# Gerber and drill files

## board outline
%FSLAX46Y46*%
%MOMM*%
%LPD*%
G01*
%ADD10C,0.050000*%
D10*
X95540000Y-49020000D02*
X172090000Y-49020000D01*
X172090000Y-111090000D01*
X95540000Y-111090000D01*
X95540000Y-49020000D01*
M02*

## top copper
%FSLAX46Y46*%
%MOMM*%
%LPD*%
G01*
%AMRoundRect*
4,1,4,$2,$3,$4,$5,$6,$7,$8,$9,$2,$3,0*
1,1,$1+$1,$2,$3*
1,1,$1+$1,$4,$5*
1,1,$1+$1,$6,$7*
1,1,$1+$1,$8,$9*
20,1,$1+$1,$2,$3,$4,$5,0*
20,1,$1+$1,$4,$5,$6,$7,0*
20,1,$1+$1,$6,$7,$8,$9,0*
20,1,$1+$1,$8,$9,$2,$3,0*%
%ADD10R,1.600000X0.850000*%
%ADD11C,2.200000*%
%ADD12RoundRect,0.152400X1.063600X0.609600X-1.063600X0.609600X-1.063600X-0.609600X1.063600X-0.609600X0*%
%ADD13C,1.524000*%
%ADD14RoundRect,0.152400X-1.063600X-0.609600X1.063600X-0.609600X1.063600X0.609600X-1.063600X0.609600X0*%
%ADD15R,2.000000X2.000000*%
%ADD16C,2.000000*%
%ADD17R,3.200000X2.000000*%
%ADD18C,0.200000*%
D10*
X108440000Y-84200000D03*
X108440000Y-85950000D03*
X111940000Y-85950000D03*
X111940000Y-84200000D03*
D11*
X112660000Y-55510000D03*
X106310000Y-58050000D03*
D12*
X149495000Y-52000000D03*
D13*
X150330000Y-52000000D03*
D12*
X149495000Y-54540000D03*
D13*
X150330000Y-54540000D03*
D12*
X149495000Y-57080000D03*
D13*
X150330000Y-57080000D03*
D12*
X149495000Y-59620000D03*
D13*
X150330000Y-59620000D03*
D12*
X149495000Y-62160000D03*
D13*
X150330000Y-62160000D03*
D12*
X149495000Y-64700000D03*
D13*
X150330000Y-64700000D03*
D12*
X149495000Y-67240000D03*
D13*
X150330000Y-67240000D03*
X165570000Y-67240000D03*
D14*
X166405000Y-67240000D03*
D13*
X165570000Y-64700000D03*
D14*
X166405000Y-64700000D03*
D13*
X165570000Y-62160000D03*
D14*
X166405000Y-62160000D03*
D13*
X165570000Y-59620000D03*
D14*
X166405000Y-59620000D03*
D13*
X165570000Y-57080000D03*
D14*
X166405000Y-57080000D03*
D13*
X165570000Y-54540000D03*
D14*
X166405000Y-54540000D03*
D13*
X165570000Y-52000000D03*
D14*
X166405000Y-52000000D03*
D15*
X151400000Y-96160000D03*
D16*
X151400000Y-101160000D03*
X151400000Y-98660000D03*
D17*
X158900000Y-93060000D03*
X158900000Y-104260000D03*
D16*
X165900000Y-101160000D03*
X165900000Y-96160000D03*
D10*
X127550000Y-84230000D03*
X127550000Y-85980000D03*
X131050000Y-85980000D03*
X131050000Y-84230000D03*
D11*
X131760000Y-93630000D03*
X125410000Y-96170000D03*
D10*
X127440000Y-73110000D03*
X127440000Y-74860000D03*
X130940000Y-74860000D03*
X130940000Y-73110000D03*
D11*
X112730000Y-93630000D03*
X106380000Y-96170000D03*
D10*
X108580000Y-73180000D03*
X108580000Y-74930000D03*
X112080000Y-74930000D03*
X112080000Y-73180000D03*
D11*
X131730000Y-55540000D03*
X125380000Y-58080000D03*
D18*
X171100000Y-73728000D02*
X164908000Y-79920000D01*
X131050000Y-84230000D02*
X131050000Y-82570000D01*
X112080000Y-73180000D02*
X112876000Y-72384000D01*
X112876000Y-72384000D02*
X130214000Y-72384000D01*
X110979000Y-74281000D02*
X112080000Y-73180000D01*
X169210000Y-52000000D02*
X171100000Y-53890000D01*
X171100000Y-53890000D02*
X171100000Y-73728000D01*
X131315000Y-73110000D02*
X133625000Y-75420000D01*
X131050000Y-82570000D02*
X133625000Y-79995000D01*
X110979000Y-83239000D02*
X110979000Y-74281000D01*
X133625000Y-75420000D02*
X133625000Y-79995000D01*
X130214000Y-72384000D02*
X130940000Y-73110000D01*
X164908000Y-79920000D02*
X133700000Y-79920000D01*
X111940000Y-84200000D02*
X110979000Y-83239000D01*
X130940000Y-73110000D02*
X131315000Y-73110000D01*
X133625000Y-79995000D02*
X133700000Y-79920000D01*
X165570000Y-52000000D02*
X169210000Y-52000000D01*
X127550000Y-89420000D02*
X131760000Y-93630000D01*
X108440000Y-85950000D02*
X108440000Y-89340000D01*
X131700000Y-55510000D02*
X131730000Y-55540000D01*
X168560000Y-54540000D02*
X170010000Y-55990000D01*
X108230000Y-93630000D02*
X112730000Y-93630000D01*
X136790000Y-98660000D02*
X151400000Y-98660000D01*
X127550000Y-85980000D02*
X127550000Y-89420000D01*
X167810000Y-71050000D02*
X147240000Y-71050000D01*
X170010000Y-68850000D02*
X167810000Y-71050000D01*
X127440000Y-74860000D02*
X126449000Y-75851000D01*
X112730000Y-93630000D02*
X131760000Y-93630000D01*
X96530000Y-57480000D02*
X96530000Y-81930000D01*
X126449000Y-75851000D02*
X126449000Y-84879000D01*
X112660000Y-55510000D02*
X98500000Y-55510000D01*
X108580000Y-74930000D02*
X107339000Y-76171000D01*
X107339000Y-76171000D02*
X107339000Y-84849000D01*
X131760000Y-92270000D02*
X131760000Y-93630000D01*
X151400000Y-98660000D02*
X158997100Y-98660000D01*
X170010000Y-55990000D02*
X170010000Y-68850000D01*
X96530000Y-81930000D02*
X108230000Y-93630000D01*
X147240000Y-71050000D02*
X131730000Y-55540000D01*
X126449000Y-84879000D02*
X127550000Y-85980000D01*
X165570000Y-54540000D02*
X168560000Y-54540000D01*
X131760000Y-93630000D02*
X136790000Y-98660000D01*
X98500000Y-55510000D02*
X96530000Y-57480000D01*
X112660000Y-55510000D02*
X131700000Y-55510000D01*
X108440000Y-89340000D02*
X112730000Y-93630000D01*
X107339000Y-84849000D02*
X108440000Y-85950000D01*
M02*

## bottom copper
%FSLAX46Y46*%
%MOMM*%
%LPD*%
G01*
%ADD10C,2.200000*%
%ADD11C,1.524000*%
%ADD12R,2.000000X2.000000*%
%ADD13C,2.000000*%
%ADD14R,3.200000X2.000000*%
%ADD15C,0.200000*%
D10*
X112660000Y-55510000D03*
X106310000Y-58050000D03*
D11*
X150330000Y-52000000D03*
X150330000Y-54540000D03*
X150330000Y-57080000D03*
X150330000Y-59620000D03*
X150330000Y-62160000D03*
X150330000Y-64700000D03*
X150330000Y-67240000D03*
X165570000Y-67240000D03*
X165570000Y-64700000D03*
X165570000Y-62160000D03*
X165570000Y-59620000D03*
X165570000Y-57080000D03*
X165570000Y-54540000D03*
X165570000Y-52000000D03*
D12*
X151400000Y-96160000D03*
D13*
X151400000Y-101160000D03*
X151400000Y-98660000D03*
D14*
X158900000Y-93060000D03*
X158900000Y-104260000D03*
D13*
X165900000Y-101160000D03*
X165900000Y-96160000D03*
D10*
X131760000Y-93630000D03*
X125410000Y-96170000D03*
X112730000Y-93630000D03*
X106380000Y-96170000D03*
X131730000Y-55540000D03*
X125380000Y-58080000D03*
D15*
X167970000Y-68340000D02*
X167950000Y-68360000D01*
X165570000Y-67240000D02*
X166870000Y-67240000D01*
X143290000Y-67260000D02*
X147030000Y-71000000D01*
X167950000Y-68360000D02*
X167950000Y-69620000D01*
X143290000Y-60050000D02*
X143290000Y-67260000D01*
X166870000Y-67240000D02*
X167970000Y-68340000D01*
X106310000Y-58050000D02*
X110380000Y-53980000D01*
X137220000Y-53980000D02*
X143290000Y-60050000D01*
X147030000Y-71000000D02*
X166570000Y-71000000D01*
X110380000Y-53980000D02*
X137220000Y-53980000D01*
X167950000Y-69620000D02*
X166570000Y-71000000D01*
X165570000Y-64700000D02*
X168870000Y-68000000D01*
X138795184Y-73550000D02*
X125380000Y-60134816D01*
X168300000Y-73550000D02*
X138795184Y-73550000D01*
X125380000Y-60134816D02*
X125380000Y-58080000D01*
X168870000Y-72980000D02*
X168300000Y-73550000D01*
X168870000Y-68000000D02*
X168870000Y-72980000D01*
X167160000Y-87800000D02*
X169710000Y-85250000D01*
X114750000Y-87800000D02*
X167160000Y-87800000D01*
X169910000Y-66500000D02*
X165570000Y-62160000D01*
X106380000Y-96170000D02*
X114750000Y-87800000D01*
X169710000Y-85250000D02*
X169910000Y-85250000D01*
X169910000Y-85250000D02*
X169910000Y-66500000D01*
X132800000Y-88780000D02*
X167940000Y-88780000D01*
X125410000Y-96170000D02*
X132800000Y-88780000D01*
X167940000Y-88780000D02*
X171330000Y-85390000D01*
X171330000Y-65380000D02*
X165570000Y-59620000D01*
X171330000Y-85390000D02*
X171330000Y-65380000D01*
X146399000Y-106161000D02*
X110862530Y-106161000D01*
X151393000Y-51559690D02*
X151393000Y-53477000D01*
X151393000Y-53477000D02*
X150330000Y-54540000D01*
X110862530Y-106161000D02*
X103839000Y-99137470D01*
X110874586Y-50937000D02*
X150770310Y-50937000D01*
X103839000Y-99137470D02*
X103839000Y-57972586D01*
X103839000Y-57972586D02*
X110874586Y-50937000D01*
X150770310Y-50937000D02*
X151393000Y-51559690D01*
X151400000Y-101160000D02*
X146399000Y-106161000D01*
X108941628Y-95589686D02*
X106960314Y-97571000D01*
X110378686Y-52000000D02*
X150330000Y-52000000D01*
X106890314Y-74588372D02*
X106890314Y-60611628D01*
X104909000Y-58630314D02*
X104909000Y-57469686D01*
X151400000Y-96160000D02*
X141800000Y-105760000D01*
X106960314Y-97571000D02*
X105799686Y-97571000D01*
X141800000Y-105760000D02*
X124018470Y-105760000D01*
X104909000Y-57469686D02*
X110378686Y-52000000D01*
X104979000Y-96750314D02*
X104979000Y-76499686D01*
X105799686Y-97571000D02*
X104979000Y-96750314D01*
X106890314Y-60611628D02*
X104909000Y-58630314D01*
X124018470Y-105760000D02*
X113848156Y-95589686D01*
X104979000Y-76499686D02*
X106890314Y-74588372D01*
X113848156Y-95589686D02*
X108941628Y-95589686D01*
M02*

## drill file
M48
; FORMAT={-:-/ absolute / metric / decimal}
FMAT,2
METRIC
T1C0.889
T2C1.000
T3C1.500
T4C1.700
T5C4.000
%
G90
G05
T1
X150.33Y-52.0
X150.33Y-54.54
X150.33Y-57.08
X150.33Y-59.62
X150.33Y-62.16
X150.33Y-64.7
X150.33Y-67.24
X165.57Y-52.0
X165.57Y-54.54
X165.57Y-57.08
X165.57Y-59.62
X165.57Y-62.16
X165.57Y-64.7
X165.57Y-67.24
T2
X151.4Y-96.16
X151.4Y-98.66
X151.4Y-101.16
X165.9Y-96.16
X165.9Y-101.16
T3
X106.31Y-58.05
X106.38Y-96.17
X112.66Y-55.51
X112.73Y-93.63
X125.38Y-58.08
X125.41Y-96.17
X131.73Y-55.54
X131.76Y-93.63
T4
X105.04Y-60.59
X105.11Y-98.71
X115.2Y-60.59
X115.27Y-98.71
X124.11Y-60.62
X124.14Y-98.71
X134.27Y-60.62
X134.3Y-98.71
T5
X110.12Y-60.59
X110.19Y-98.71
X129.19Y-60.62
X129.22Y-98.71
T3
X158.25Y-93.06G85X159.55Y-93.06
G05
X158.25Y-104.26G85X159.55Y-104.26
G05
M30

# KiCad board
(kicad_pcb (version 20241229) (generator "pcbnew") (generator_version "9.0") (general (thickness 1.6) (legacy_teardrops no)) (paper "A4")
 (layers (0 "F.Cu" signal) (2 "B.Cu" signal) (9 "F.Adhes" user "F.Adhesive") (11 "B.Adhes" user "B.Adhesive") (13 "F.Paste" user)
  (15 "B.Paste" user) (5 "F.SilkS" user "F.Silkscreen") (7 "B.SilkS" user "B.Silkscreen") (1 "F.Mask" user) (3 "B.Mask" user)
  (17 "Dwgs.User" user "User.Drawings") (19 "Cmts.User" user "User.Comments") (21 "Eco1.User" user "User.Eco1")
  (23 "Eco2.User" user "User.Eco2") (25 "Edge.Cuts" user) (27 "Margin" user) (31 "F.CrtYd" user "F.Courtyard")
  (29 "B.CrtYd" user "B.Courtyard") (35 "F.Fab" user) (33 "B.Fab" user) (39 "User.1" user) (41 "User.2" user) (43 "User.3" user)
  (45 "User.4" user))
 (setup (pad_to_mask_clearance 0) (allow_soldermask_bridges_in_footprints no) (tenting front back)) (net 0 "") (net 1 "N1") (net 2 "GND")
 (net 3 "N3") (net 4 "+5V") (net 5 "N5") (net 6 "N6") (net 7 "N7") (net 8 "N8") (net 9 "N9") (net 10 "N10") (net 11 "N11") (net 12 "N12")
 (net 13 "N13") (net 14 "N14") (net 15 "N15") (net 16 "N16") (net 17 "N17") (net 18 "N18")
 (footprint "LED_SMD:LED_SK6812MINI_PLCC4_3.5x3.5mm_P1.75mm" (layer "F.Cu") (at 110.19 85.075)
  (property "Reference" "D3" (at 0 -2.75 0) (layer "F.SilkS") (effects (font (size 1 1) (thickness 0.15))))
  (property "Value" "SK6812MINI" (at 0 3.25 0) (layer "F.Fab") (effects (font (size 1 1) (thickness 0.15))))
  (pad "1" smd rect (at -1.75 -0.875) (size 1.6 0.85) (layers "F.Cu" "F.Mask" "F.Paste") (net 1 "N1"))
  (pad "2" smd rect (at -1.75 0.875) (size 1.6 0.85) (layers "F.Cu" "F.Mask" "F.Paste") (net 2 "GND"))
  (pad "3" smd rect (at 1.75 0.875) (size 1.6 0.85) (layers "F.Cu" "F.Mask" "F.Paste") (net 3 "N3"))
  (pad "4" smd rect (at 1.75 -0.875) (size 1.6 0.85) (layers "F.Cu" "F.Mask" "F.Paste") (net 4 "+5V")))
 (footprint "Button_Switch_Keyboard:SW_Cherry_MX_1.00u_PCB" (layer "F.Cu") (at 112.66 55.51)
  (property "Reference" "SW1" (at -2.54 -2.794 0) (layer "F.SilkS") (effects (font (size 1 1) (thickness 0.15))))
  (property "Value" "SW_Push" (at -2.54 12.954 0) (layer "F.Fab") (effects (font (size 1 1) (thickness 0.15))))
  (pad "" np_thru_hole circle (at -7.62 5.08) (size 1.7 1.7) (drill 1.7) (layers "*.Cu" "*.Mask"))
  (pad "" np_thru_hole circle (at -2.54 5.08) (size 4 4) (drill 4) (layers "*.Cu" "*.Mask"))
  (pad "" np_thru_hole circle (at 2.54 5.08) (size 1.7 1.7) (drill 1.7) (layers "*.Cu" "*.Mask"))
  (pad "1" thru_hole circle (at 0 0) (size 2.2 2.2) (drill 1.5) (layers "*.Cu" "*.Mask") (remove_unused_layers no) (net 2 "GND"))
  (pad "2" thru_hole circle (at -6.35 2.54) (size 2.2 2.2) (drill 1.5) (layers "*.Cu" "*.Mask") (remove_unused_layers no) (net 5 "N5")))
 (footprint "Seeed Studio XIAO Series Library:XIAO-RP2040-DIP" (layer "F.Cu") (at 157.95 59.62)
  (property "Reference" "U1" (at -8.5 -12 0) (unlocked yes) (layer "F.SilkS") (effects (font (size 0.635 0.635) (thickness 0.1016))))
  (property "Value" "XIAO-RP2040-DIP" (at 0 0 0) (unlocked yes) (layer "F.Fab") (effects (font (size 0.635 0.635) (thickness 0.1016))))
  (pad "1" smd roundrect (at -8.455 -7.62 180) (size 2.432 1.524) (layers "F.Cu" "F.Mask") (roundrect_rratio 0.1) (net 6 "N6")
   (thermal_bridge_angle 45))
  (pad "1" thru_hole circle (at -7.62 -7.62 180) (size 1.524 1.524) (drill 0.889) (layers "*.Cu" "*.Mask") (remove_unused_layers no)
   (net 6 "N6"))
  (pad "2" smd roundrect (at -8.455 -5.08 180) (size 2.432 1.524) (layers "F.Cu" "F.Mask") (roundrect_rratio 0.1) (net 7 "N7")
   (thermal_bridge_angle 45))
  (pad "2" thru_hole circle (at -7.62 -5.08 180) (size 1.524 1.524) (drill 0.889) (layers "*.Cu" "*.Mask") (remove_unused_layers no)
   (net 7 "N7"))
  (pad "3" smd roundrect (at -8.455 -2.54 180) (size 2.432 1.524) (layers "F.Cu" "F.Mask") (roundrect_rratio 0.1) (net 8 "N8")
   (thermal_bridge_angle 45))
  (pad "3" thru_hole circle (at -7.62 -2.54 180) (size 1.524 1.524) (drill 0.889) (layers "*.Cu" "*.Mask") (remove_unused_layers no)
   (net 8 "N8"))
  (pad "4" smd roundrect (at -8.455 0 180) (size 2.432 1.524) (layers "F.Cu" "F.Mask") (roundrect_rratio 0.1) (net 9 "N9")
   (thermal_bridge_angle 45))
  (pad "4" thru_hole circle (at -7.62 0 180) (size 1.524 1.524) (drill 0.889) (layers "*.Cu" "*.Mask") (remove_unused_layers no)
   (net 9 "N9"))
  (pad "5" smd roundrect (at -8.455 2.54 180) (size 2.432 1.524) (layers "F.Cu" "F.Mask") (roundrect_rratio 0.1) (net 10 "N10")
   (thermal_bridge_angle 45))
  (pad "5" thru_hole circle (at -7.62 2.54 180) (size 1.524 1.524) (drill 0.889) (layers "*.Cu" "*.Mask") (remove_unused_layers no)
   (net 10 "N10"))
  (pad "6" smd roundrect (at -8.455 5.08 180) (size 2.432 1.524) (layers "F.Cu" "F.Mask") (roundrect_rratio 0.1) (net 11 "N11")
   (thermal_bridge_angle 45))
  (pad "6" thru_hole circle (at -7.62 5.08 180) (size 1.524 1.524) (drill 0.889) (layers "*.Cu" "*.Mask") (remove_unused_layers no)
   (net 11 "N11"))
  (pad "7" smd roundrect (at -8.455 7.62 180) (size 2.432 1.524) (layers "F.Cu" "F.Mask") (roundrect_rratio 0.1) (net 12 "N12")
   (thermal_bridge_angle 45))
  (pad "7" thru_hole circle (at -7.62 7.62 180) (size 1.524 1.524) (drill 0.889) (layers "*.Cu" "*.Mask") (remove_unused_layers no)
   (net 12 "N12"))
  (pad "8" thru_hole circle (at 7.62 7.62) (size 1.524 1.524) (drill 0.889) (layers "*.Cu" "*.Mask") (remove_unused_layers no) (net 5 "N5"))
  (pad "8" smd roundrect (at 8.455 7.62) (size 2.432 1.524) (layers "F.Cu" "F.Mask") (roundrect_rratio 0.1) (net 5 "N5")
   (thermal_bridge_angle 45))
  (pad "9" thru_hole circle (at 7.62 5.08) (size 1.524 1.524) (drill 0.889) (layers "*.Cu" "*.Mask") (remove_unused_layers no)
   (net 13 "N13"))
  (pad "9" smd roundrect (at 8.455 5.08) (size 2.432 1.524) (layers "F.Cu" "F.Mask") (roundrect_rratio 0.1) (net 13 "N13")
   (thermal_bridge_angle 45))
  (pad "10" thru_hole circle (at 7.62 2.54) (size 1.524 1.524) (drill 0.889) (layers "*.Cu" "*.Mask") (remove_unused_layers no)
   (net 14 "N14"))
  (pad "10" smd roundrect (at 8.455 2.54) (size 2.432 1.524) (layers "F.Cu" "F.Mask") (roundrect_rratio 0.1) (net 14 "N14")
   (thermal_bridge_angle 45))
  (pad "11" thru_hole circle (at 7.62 0) (size 1.524 1.524) (drill 0.889) (layers "*.Cu" "*.Mask") (remove_unused_layers no) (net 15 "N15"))
  (pad "11" smd roundrect (at 8.455 0) (size 2.432 1.524) (layers "F.Cu" "F.Mask") (roundrect_rratio 0.1) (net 15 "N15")
   (thermal_bridge_angle 45))
  (pad "12" thru_hole circle (at 7.62 -2.54) (size 1.524 1.524) (drill 0.889) (layers "*.Cu" "*.Mask") (remove_unused_layers no)
   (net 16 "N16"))
  (pad "12" smd roundrect (at 8.455 -2.54) (size 2.432 1.524) (layers "F.Cu" "F.Mask") (roundrect_rratio 0.1) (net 16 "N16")
   (thermal_bridge_angle 45))
  (pad "13" thru_hole circle (at 7.62 -5.08) (size 1.524 1.524) (drill 0.889) (layers "*.Cu" "*.Mask") (remove_unused_layers no)
   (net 2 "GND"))
  (pad "13" smd roundrect (at 8.455 -5.08) (size 2.432 1.524) (layers "F.Cu" "F.Mask") (roundrect_rratio 0.1) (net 2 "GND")
   (thermal_bridge_angle 45))
  (pad "14" thru_hole circle (at 7.62 -7.62) (size 1.524 1.524) (drill 0.889) (layers "*.Cu" "*.Mask") (remove_unused_layers no)
   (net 4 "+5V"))
  (pad "14" smd roundrect (at 8.455 -7.62) (size 2.432 1.524) (layers "F.Cu" "F.Mask") (roundrect_rratio 0.1) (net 4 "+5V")
   (thermal_bridge_angle 45)))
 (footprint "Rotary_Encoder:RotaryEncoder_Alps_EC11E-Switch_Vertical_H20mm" (layer "F.Cu") (at 151.4 96.16)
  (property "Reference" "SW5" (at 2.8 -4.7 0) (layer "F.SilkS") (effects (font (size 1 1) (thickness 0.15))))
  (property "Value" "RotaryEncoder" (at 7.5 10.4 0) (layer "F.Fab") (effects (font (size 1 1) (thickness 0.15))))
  (pad "A" thru_hole rect (at 0 0) (size 2 2) (drill 1) (layers "*.Cu" "*.Mask") (remove_unused_layers no) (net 6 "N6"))
  (pad "B" thru_hole circle (at 0 5) (size 2 2) (drill 1) (layers "*.Cu" "*.Mask") (remove_unused_layers no) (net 7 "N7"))
  (pad "C" thru_hole circle (at 0 2.5) (size 2 2) (drill 1) (layers "*.Cu" "*.Mask") (remove_unused_layers no) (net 2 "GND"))
  (pad "MP" thru_hole rect (at 7.5 -3.1) (size 3.2 2) (drill oval 2.8 1.5) (layers "*.Cu" "*.Mask") (remove_unused_layers no))
  (pad "MP" thru_hole rect (at 7.5 8.1) (size 3.2 2) (drill oval 2.8 1.5) (layers "*.Cu" "*.Mask") (remove_unused_layers no))
  (pad "S1" thru_hole circle (at 14.5 5) (size 2 2) (drill 1) (layers "*.Cu" "*.Mask") (remove_unused_layers no))
  (pad "S2" thru_hole circle (at 14.5 0) (size 2 2) (drill 1) (layers "*.Cu" "*.Mask") (remove_unused_layers no)))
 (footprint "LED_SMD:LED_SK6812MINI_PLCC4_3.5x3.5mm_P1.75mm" (layer "F.Cu") (at 129.3 85.105)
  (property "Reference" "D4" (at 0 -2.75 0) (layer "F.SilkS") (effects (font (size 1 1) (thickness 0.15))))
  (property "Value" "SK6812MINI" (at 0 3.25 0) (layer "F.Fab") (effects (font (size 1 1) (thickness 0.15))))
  (pad "1" smd rect (at -1.75 -0.875) (size 1.6 0.85) (layers "F.Cu" "F.Mask" "F.Paste") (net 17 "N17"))
  (pad "2" smd rect (at -1.75 0.875) (size 1.6 0.85) (layers "F.Cu" "F.Mask" "F.Paste") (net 2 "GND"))
  (pad "3" smd rect (at 1.75 0.875) (size 1.6 0.85) (layers "F.Cu" "F.Mask" "F.Paste") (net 1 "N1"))
  (pad "4" smd rect (at 1.75 -0.875) (size 1.6 0.85) (layers "F.Cu" "F.Mask" "F.Paste") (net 4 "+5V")))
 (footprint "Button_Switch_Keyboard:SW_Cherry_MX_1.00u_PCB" (layer "F.Cu") (at 131.76 93.63)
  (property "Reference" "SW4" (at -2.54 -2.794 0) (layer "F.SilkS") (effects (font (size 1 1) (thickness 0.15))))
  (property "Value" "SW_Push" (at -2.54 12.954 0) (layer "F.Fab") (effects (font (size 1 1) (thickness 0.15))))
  (pad "" np_thru_hole circle (at -7.62 5.08) (size 1.7 1.7) (drill 1.7) (layers "*.Cu" "*.Mask"))
  (pad "" np_thru_hole circle (at -2.54 5.08) (size 4 4) (drill 4) (layers "*.Cu" "*.Mask"))
  (pad "" np_thru_hole circle (at 2.54 5.08) (size 1.7 1.7) (drill 1.7) (layers "*.Cu" "*.Mask"))
  (pad "1" thru_hole circle (at 0 0) (size 2.2 2.2) (drill 1.5) (layers "*.Cu" "*.Mask") (remove_unused_layers no) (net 2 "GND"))
  (pad "2" thru_hole circle (at -6.35 2.54) (size 2.2 2.2) (drill 1.5) (layers "*.Cu" "*.Mask") (remove_unused_layers no) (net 15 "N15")))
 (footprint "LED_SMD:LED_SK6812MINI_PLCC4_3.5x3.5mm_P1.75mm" (layer "F.Cu") (at 129.19 73.985)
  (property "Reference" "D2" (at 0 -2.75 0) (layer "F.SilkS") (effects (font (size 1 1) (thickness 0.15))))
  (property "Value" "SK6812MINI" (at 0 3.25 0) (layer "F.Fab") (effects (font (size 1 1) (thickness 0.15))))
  (pad "1" smd rect (at -1.75 -0.875) (size 1.6 0.85) (layers "F.Cu" "F.Mask" "F.Paste") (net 3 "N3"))
  (pad "2" smd rect (at -1.75 0.875) (size 1.6 0.85) (layers "F.Cu" "F.Mask" "F.Paste") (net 2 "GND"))
  (pad "3" smd rect (at 1.75 0.875) (size 1.6 0.85) (layers "F.Cu" "F.Mask" "F.Paste") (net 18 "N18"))
  (pad "4" smd rect (at 1.75 -0.875) (size 1.6 0.85) (layers "F.Cu" "F.Mask" "F.Paste") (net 4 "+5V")))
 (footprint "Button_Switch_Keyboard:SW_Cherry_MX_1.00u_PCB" (layer "F.Cu") (at 112.73 93.63)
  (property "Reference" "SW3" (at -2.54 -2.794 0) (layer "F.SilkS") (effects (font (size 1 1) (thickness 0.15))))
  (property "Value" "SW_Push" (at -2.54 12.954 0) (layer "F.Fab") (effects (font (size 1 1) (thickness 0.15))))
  (pad "" np_thru_hole circle (at -7.62 5.08) (size 1.7 1.7) (drill 1.7) (layers "*.Cu" "*.Mask"))
  (pad "" np_thru_hole circle (at -2.54 5.08) (size 4 4) (drill 4) (layers "*.Cu" "*.Mask"))
  (pad "" np_thru_hole circle (at 2.54 5.08) (size 1.7 1.7) (drill 1.7) (layers "*.Cu" "*.Mask"))
  (pad "1" thru_hole circle (at 0 0) (size 2.2 2.2) (drill 1.5) (layers "*.Cu" "*.Mask") (remove_unused_layers no) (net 2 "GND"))
  (pad "2" thru_hole circle (at -6.35 2.54) (size 2.2 2.2) (drill 1.5) (layers "*.Cu" "*.Mask") (remove_unused_layers no) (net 14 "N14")))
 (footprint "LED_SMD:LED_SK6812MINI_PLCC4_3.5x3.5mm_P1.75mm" (layer "F.Cu") (at 110.33 74.055)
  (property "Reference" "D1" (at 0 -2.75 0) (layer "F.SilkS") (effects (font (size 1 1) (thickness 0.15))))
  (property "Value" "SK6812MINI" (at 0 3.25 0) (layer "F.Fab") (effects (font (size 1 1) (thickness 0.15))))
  (pad "1" smd rect (at -1.75 -0.875) (size 1.6 0.85) (layers "F.Cu" "F.Mask" "F.Paste") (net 18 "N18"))
  (pad "2" smd rect (at -1.75 0.875) (size 1.6 0.85) (layers "F.Cu" "F.Mask" "F.Paste") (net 2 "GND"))
  (pad "3" smd rect (at 1.75 0.875) (size 1.6 0.85) (layers "F.Cu" "F.Mask" "F.Paste") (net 10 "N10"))
  (pad "4" smd rect (at 1.75 -0.875) (size 1.6 0.85) (layers "F.Cu" "F.Mask" "F.Paste") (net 4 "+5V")))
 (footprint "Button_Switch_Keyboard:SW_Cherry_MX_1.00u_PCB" (layer "F.Cu") (at 131.73 55.54)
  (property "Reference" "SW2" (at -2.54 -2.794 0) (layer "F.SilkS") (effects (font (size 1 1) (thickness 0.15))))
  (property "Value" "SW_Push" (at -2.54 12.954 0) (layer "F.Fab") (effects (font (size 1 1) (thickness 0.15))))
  (pad "" np_thru_hole circle (at -7.62 5.08) (size 1.7 1.7) (drill 1.7) (layers "*.Cu" "*.Mask"))
  (pad "" np_thru_hole circle (at -2.54 5.08) (size 4 4) (drill 4) (layers "*.Cu" "*.Mask"))
  (pad "" np_thru_hole circle (at 2.54 5.08) (size 1.7 1.7) (drill 1.7) (layers "*.Cu" "*.Mask"))
  (pad "1" thru_hole circle (at 0 0) (size 2.2 2.2) (drill 1.5) (layers "*.Cu" "*.Mask") (remove_unused_layers no) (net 2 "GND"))
  (pad "2" thru_hole circle (at -6.35 2.54) (size 2.2 2.2) (drill 1.5) (layers "*.Cu" "*.Mask") (remove_unused_layers no) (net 13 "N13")))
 (gr_rect (start 95.54 49.02) (end 172.09 111.09) (stroke (width 0.05) (type default)) (fill no) (layer "Edge.Cuts"))
 (segment (start 171.1 73.728) (end 164.908 79.92) (width 0.2) (layer "F.Cu") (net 4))
 (segment (start 131.05 84.23) (end 131.05 82.57) (width 0.2) (layer "F.Cu") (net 4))
 (segment (start 112.08 73.18) (end 112.876 72.384) (width 0.2) (layer "F.Cu") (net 4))
 (segment (start 112.876 72.384) (end 130.214 72.384) (width 0.2) (layer "F.Cu") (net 4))
 (segment (start 110.979 74.281) (end 112.08 73.18) (width 0.2) (layer "F.Cu") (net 4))
 (segment (start 169.21 52) (end 171.1 53.89) (width 0.2) (layer "F.Cu") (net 4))
 (segment (start 171.1 53.89) (end 171.1 73.728) (width 0.2) (layer "F.Cu") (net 4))
 (segment (start 131.315 73.11) (end 133.625 75.42) (width 0.2) (layer "F.Cu") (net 4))
 (segment (start 131.05 82.57) (end 133.625 79.995) (width 0.2) (layer "F.Cu") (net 4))
 (segment (start 110.979 83.239) (end 110.979 74.281) (width 0.2) (layer "F.Cu") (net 4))
 (segment (start 133.625 75.42) (end 133.625 79.995) (width 0.2) (layer "F.Cu") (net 4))
 (segment (start 130.214 72.384) (end 130.94 73.11) (width 0.2) (layer "F.Cu") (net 4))
 (segment (start 164.908 79.92) (end 133.7 79.92) (width 0.2) (layer "F.Cu") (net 4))
 (segment (start 111.94 84.2) (end 110.979 83.239) (width 0.2) (layer "F.Cu") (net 4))
 (segment (start 130.94 73.11) (end 131.315 73.11) (width 0.2) (layer "F.Cu") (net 4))
 (segment (start 133.625 79.995) (end 133.7 79.92) (width 0.2) (layer "F.Cu") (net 4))
 (segment (start 165.57 52) (end 169.21 52) (width 0.2) (layer "F.Cu") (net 4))
 (segment (start 127.55 89.42) (end 131.76 93.63) (width 0.2) (layer "F.Cu") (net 2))
 (segment (start 108.44 85.95) (end 108.44 89.34) (width 0.2) (layer "F.Cu") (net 2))
 (segment (start 131.7 55.51) (end 131.73 55.54) (width 0.2) (layer "F.Cu") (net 2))
 (segment (start 168.56 54.54) (end 170.01 55.99) (width 0.2) (layer "F.Cu") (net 2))
 (segment (start 108.23 93.63) (end 112.73 93.63) (width 0.2) (layer "F.Cu") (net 2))
 (segment (start 136.79 98.66) (end 151.4 98.66) (width 0.2) (layer "F.Cu") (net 2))
 (segment (start 127.55 85.98) (end 127.55 89.42) (width 0.2) (layer "F.Cu") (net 2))
 (segment (start 167.81 71.05) (end 147.24 71.05) (width 0.2) (layer "F.Cu") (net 2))
 (segment (start 170.01 68.85) (end 167.81 71.05) (width 0.2) (layer "F.Cu") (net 2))
 (segment (start 127.44 74.86) (end 126.449 75.851) (width 0.2) (layer "F.Cu") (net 2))
 (segment (start 112.73 93.63) (end 131.76 93.63) (width 0.2) (layer "F.Cu") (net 2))
 (segment (start 96.53 57.48) (end 96.53 81.93) (width 0.2) (layer "F.Cu") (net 2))
 (segment (start 126.449 75.851) (end 126.449 84.879) (width 0.2) (layer "F.Cu") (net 2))
 (segment (start 112.66 55.51) (end 98.5 55.51) (width 0.2) (layer "F.Cu") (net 2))
 (segment (start 108.58 74.93) (end 107.339 76.171) (width 0.2) (layer "F.Cu") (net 2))
 (segment (start 107.339 76.171) (end 107.339 84.849) (width 0.2) (layer "F.Cu") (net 2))
 (segment (start 131.76 92.27) (end 131.76 93.63) (width 0.2) (layer "F.Cu") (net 2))
 (segment (start 151.4 98.66) (end 158.9971 98.66) (width 0.2) (layer "F.Cu") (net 2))
 (segment (start 170.01 55.99) (end 170.01 68.85) (width 0.2) (layer "F.Cu") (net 2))
 (segment (start 96.53 81.93) (end 108.23 93.63) (width 0.2) (layer "F.Cu") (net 2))
 (segment (start 147.24 71.05) (end 131.73 55.54) (width 0.2) (layer "F.Cu") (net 2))
 (segment (start 126.449 84.879) (end 127.55 85.98) (width 0.2) (layer "F.Cu") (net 2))
 (segment (start 165.57 54.54) (end 168.56 54.54) (width 0.2) (layer "F.Cu") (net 2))
 (segment (start 131.76 93.63) (end 136.79 98.66) (width 0.2) (layer "F.Cu") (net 2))
 (segment (start 98.5 55.51) (end 96.53 57.48) (width 0.2) (layer "F.Cu") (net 2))
 (segment (start 112.66 55.51) (end 131.7 55.51) (width 0.2) (layer "F.Cu") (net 2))
 (segment (start 108.44 89.34) (end 112.73 93.63) (width 0.2) (layer "F.Cu") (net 2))
 (segment (start 107.339 84.849) (end 108.44 85.95) (width 0.2) (layer "F.Cu") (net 2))
 (segment (start 167.97 68.34) (end 167.95 68.36) (width 0.2) (layer "B.Cu") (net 5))
 (segment (start 165.57 67.24) (end 166.87 67.24) (width 0.2) (layer "B.Cu") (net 5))
 (segment (start 143.29 67.26) (end 147.03 71) (width 0.2) (layer "B.Cu") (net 5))
 (segment (start 167.95 68.36) (end 167.95 69.62) (width 0.2) (layer "B.Cu") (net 5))
 (segment (start 143.29 60.05) (end 143.29 67.26) (width 0.2) (layer "B.Cu") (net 5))
 (segment (start 166.87 67.24) (end 167.97 68.34) (width 0.2) (layer "B.Cu") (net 5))
 (segment (start 106.31 58.05) (end 110.38 53.98) (width 0.2) (layer "B.Cu") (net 5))
 (segment (start 137.22 53.98) (end 143.29 60.05) (width 0.2) (layer "B.Cu") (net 5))
 (segment (start 147.03 71) (end 166.57 71) (width 0.2) (layer "B.Cu") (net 5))
 (segment (start 110.38 53.98) (end 137.22 53.98) (width 0.2) (layer "B.Cu") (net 5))
 (segment (start 167.95 69.62) (end 166.57 71) (width 0.2) (layer "B.Cu") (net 5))
 (segment (start 165.57 64.7) (end 168.87 68) (width 0.2) (layer "B.Cu") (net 13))
 (segment (start 138.795184 73.55) (end 125.38 60.134816) (width 0.2) (layer "B.Cu") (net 13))
 (segment (start 168.3 73.55) (end 138.795184 73.55) (width 0.2) (layer "B.Cu") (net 13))
 (segment (start 125.38 60.134816) (end 125.38 58.08) (width 0.2) (layer "B.Cu") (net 13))
 (segment (start 168.87 72.98) (end 168.3 73.55) (width 0.2) (layer "B.Cu") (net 13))
 (segment (start 168.87 68) (end 168.87 72.98) (width 0.2) (layer "B.Cu") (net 13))
 (segment (start 167.16 87.8) (end 169.71 85.25) (width 0.2) (layer "B.Cu") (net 14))
 (segment (start 114.75 87.8) (end 167.16 87.8) (width 0.2) (layer "B.Cu") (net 14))
 (segment (start 169.91 66.5) (end 165.57 62.16) (width 0.2) (layer "B.Cu") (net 14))
 (segment (start 106.38 96.17) (end 114.75 87.8) (width 0.2) (layer "B.Cu") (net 14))
 (segment (start 169.71 85.25) (end 169.91 85.25) (width 0.2) (layer "B.Cu") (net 14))
 (segment (start 169.91 85.25) (end 169.91 66.5) (width 0.2) (layer "B.Cu") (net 14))
 (segment (start 132.8 88.78) (end 167.94 88.78) (width 0.2) (layer "B.Cu") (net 15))
 (segment (start 125.41 96.17) (end 132.8 88.78) (width 0.2) (layer "B.Cu") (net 15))
 (segment (start 167.94 88.78) (end 171.33 85.39) (width 0.2) (layer "B.Cu") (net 15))
 (segment (start 171.33 65.38) (end 165.57 59.62) (width 0.2) (layer "B.Cu") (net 15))
 (segment (start 171.33 85.39) (end 171.33 65.38) (width 0.2) (layer "B.Cu") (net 15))
 (segment (start 146.399 106.161) (end 110.86253 106.161) (width 0.2) (layer "B.Cu") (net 7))
 (segment (start 151.393 51.55969) (end 151.393 53.477) (width 0.2) (layer "B.Cu") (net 7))
 (segment (start 151.393 53.477) (end 150.33 54.54) (width 0.2) (layer "B.Cu") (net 7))
 (segment (start 110.86253 106.161) (end 103.839 99.13747) (width 0.2) (layer "B.Cu") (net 7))
 (segment (start 110.874586 50.937) (end 150.77031 50.937) (width 0.2) (layer "B.Cu") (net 7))
 (segment (start 103.839 99.13747) (end 103.839 57.972586) (width 0.2) (layer "B.Cu") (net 7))
 (segment (start 103.839 57.972586) (end 110.874586 50.937) (width 0.2) (layer "B.Cu") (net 7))
 (segment (start 150.77031 50.937) (end 151.393 51.55969) (width 0.2) (layer "B.Cu") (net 7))
 (segment (start 151.4 101.16) (end 146.399 106.161) (width 0.2) (layer "B.Cu") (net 7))
 (segment (start 108.941628 95.589686) (end 106.960314 97.571) (width 0.2) (layer "B.Cu") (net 6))
 (segment (start 110.378686 52) (end 150.33 52) (width 0.2) (layer "B.Cu") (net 6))
 (segment (start 106.890314 74.588372) (end 106.890314 60.611628) (width 0.2) (layer "B.Cu") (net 6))
 (segment (start 104.909 58.630314) (end 104.909 57.469686) (width 0.2) (layer "B.Cu") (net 6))
 (segment (start 151.4 96.16) (end 141.8 105.76) (width 0.2) (layer "B.Cu") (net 6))
 (segment (start 106.960314 97.571) (end 105.799686 97.571) (width 0.2) (layer "B.Cu") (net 6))
 (segment (start 141.8 105.76) (end 124.01847 105.76) (width 0.2) (layer "B.Cu") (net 6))
 (segment (start 104.909 57.469686) (end 110.378686 52) (width 0.2) (layer "B.Cu") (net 6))
 (segment (start 104.979 96.750314) (end 104.979 76.499686) (width 0.2) (layer "B.Cu") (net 6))
 (segment (start 105.799686 97.571) (end 104.979 96.750314) (width 0.2) (layer "B.Cu") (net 6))
 (segment (start 106.890314 60.611628) (end 104.909 58.630314) (width 0.2) (layer "B.Cu") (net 6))
 (segment (start 124.01847 105.76) (end 113.848156 95.589686) (width 0.2) (layer "B.Cu") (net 6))
 (segment (start 104.979 76.499686) (end 106.890314 74.588372) (width 0.2) (layer "B.Cu") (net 6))
 (segment (start 113.848156 95.589686) (end 108.941628 95.589686) (width 0.2) (layer "B.Cu") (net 6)))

